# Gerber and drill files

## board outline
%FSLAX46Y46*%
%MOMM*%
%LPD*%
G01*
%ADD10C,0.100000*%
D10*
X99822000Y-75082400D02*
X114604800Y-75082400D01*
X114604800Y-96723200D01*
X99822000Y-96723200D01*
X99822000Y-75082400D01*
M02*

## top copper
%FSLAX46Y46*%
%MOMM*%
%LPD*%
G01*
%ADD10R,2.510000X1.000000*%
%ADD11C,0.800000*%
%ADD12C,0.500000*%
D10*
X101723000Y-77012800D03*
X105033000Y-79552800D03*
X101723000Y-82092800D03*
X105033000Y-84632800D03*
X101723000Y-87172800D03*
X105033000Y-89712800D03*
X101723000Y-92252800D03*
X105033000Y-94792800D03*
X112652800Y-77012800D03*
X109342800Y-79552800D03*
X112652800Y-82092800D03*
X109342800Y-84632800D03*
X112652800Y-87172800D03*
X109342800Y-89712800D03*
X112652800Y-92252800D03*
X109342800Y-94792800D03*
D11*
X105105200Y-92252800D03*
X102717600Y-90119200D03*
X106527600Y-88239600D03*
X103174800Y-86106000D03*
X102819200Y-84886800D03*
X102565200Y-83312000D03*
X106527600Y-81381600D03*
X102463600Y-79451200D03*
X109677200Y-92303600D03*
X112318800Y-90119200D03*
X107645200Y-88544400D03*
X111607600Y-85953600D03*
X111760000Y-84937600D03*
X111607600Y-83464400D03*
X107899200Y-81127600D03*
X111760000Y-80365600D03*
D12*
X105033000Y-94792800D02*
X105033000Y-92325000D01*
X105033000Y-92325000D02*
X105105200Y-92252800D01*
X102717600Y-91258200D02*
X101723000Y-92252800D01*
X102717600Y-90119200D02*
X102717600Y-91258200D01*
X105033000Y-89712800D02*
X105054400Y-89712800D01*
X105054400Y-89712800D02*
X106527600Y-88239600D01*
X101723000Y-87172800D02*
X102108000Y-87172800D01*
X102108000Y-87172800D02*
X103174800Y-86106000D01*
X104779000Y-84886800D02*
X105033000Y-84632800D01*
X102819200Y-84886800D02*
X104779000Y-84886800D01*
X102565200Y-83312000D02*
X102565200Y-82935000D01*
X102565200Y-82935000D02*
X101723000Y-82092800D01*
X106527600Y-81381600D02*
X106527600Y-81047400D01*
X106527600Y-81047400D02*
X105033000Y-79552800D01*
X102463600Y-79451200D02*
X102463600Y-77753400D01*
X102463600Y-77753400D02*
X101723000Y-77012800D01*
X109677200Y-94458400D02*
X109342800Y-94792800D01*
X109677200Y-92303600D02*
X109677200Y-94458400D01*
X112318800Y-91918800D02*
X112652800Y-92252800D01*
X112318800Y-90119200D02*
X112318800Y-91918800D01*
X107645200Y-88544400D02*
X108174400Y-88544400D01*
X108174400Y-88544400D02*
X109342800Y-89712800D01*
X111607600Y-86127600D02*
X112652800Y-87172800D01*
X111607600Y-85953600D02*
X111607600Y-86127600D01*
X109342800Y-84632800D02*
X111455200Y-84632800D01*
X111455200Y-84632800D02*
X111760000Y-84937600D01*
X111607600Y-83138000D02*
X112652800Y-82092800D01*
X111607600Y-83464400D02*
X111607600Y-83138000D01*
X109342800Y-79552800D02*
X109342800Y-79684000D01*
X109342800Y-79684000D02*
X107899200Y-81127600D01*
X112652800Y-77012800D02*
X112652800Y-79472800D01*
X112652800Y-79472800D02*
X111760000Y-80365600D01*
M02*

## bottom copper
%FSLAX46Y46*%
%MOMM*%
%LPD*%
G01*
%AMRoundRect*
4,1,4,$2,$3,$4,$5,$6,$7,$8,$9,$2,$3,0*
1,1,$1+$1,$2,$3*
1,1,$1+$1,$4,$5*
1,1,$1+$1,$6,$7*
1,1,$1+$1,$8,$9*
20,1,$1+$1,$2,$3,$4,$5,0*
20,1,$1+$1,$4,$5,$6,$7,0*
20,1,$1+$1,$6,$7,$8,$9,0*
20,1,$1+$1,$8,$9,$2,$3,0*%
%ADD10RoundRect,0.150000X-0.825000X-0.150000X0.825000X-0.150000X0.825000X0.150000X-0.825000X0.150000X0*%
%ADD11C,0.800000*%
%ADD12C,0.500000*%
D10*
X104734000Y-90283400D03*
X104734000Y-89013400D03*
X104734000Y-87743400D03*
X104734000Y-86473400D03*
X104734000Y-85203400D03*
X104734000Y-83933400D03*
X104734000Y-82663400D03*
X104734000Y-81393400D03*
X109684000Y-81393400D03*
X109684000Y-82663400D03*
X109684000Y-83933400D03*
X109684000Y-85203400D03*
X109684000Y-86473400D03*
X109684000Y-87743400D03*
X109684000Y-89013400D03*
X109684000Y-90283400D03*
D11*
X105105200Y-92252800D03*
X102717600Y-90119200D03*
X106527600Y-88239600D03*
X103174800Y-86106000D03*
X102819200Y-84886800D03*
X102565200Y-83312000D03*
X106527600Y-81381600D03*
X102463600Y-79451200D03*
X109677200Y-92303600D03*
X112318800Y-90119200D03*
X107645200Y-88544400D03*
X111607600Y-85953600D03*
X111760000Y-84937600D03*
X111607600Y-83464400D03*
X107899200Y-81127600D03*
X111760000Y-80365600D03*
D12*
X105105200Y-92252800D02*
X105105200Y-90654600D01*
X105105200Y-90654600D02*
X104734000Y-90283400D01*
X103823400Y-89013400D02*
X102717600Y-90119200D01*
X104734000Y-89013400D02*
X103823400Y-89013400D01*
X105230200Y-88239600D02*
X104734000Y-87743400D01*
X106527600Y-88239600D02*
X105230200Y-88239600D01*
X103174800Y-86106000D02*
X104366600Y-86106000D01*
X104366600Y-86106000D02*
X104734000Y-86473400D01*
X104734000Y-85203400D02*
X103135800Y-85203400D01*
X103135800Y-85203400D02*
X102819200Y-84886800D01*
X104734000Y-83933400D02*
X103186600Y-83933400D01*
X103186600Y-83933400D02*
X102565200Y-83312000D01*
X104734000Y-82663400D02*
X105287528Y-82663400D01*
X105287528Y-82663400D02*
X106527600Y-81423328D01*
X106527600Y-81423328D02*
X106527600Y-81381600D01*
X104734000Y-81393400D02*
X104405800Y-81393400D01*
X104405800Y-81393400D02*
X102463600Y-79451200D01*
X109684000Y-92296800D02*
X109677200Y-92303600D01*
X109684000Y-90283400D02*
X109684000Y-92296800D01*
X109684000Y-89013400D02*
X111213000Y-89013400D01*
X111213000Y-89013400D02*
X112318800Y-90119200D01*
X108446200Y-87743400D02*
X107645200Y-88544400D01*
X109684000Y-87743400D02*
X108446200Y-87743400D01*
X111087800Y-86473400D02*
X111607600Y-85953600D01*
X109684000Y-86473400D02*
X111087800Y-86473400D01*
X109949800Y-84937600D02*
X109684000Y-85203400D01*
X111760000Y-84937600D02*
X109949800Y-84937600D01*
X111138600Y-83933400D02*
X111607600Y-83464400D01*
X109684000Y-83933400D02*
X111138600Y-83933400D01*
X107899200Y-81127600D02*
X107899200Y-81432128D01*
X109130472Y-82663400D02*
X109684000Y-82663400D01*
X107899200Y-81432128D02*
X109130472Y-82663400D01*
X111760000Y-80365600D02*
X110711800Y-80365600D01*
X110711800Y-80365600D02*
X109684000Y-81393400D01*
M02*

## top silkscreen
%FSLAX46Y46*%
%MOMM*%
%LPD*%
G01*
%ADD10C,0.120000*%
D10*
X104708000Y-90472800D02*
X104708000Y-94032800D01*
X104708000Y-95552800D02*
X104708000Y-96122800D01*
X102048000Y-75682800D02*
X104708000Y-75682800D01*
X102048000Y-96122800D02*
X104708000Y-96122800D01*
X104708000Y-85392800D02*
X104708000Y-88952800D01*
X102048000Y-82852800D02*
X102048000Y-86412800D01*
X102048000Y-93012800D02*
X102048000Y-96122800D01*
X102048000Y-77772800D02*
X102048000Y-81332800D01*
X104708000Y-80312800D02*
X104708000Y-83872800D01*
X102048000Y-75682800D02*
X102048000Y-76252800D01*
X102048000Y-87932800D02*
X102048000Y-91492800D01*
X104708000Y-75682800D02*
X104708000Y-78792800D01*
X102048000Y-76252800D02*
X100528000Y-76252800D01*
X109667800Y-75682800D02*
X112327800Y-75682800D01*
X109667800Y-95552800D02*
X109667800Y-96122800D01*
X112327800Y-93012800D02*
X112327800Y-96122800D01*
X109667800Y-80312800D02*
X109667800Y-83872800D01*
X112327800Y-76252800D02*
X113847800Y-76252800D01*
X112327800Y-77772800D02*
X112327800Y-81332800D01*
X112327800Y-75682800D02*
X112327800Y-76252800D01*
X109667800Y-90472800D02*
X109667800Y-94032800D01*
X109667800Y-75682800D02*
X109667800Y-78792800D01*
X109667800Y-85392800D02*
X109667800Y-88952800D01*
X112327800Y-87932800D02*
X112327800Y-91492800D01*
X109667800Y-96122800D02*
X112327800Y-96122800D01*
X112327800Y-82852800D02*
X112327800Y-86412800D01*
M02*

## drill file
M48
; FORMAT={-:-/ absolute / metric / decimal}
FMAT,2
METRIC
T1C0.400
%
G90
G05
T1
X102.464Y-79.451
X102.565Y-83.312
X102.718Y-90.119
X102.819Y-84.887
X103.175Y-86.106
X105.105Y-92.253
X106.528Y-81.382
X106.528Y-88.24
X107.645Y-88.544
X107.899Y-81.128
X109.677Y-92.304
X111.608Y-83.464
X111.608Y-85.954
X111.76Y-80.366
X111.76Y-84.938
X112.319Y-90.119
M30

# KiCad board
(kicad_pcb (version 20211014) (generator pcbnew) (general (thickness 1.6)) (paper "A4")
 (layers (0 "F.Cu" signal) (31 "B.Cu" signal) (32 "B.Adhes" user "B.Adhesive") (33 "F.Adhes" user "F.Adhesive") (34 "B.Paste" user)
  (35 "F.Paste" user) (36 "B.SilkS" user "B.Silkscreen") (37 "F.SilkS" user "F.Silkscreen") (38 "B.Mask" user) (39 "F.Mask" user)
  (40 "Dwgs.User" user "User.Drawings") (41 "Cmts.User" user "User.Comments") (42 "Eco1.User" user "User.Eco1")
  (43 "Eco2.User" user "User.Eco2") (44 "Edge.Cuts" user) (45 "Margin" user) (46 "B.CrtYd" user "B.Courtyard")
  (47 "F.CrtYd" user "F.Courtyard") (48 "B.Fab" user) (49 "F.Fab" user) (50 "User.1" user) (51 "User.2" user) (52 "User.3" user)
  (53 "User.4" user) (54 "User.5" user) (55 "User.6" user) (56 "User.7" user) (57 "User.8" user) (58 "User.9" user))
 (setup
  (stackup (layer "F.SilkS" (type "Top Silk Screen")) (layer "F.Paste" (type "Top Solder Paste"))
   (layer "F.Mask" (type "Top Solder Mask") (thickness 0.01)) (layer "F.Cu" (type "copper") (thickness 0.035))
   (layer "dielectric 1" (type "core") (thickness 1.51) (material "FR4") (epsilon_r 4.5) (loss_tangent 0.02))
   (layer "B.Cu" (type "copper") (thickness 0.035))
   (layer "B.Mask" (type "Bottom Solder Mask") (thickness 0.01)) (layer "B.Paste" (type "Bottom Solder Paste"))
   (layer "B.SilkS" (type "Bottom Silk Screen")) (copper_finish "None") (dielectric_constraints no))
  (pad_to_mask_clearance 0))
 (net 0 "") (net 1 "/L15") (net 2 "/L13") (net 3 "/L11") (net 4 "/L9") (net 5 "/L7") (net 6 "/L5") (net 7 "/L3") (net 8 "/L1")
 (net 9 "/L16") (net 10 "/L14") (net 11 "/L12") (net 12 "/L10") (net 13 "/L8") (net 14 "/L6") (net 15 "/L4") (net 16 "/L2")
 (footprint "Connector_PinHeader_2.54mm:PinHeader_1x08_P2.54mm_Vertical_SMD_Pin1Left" (layer "F.Cu") (at 103.378 85.9028)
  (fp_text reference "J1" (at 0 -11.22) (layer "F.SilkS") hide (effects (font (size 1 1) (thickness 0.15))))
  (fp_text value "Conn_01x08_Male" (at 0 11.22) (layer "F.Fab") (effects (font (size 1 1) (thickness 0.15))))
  (fp_line (start 1.33 4.57) (end 1.33 8.13) (layer "F.SilkS") (width 0.12))
  (fp_line (start 1.33 9.65) (end 1.33 10.22) (layer "F.SilkS") (width 0.12))
  (fp_line (start -1.33 -10.22) (end 1.33 -10.22) (layer "F.SilkS") (width 0.12))
  (fp_line (start -1.33 10.22) (end 1.33 10.22) (layer "F.SilkS") (width 0.12))
  (fp_line (start 1.33 -0.51) (end 1.33 3.05) (layer "F.SilkS") (width 0.12))
  (fp_line (start -1.33 -3.05) (end -1.33 0.51) (layer "F.SilkS") (width 0.12))
  (fp_line (start -1.33 7.11) (end -1.33 10.22) (layer "F.SilkS") (width 0.12))
  (fp_line (start -1.33 -8.13) (end -1.33 -4.57) (layer "F.SilkS") (width 0.12))
  (fp_line (start 1.33 -5.59) (end 1.33 -2.03) (layer "F.SilkS") (width 0.12))
  (fp_line (start -1.33 -10.22) (end -1.33 -9.65) (layer "F.SilkS") (width 0.12))
  (fp_line (start -1.33 2.03) (end -1.33 5.59) (layer "F.SilkS") (width 0.12))
  (fp_line (start 1.33 -10.22) (end 1.33 -7.11) (layer "F.SilkS") (width 0.12))
  (fp_line (start -1.33 -9.65) (end -2.85 -9.65) (layer "F.SilkS") (width 0.12))
  (pad "1" smd rect (at -1.655 -8.89) (size 2.51 1) (layers "F.Cu" "F.Paste" "F.Mask") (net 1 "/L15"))
  (pad "2" smd rect (at 1.655 -6.35) (size 2.51 1) (layers "F.Cu" "F.Paste" "F.Mask") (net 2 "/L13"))
  (pad "3" smd rect (at -1.655 -3.81) (size 2.51 1) (layers "F.Cu" "F.Paste" "F.Mask") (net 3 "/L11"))
  (pad "4" smd rect (at 1.655 -1.27) (size 2.51 1) (layers "F.Cu" "F.Paste" "F.Mask") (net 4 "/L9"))
  (pad "5" smd rect (at -1.655 1.27) (size 2.51 1) (layers "F.Cu" "F.Paste" "F.Mask") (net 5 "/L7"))
  (pad "6" smd rect (at 1.655 3.81) (size 2.51 1) (layers "F.Cu" "F.Paste" "F.Mask") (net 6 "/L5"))
  (pad "7" smd rect (at -1.655 6.35) (size 2.51 1) (layers "F.Cu" "F.Paste" "F.Mask") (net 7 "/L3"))
  (pad "8" smd rect (at 1.655 8.89) (size 2.51 1) (layers "F.Cu" "F.Paste" "F.Mask") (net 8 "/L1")))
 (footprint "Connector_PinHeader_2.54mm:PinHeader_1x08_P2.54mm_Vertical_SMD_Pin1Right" (layer "F.Cu") (at 110.9978 85.9028)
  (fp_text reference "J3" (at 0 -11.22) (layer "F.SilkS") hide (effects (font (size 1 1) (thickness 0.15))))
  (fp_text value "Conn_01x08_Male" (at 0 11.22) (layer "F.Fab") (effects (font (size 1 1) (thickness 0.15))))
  (fp_line (start -1.33 -10.22) (end 1.33 -10.22) (layer "F.SilkS") (width 0.12))
  (fp_line (start -1.33 9.65) (end -1.33 10.22) (layer "F.SilkS") (width 0.12))
  (fp_line (start 1.33 7.11) (end 1.33 10.22) (layer "F.SilkS") (width 0.12))
  (fp_line (start -1.33 -5.59) (end -1.33 -2.03) (layer "F.SilkS") (width 0.12))
  (fp_line (start 1.33 -9.65) (end 2.85 -9.65) (layer "F.SilkS") (width 0.12))
  (fp_line (start 1.33 -8.13) (end 1.33 -4.57) (layer "F.SilkS") (width 0.12))
  (fp_line (start 1.33 -10.22) (end 1.33 -9.65) (layer "F.SilkS") (width 0.12))
  (fp_line (start -1.33 4.57) (end -1.33 8.13) (layer "F.SilkS") (width 0.12))
  (fp_line (start -1.33 -10.22) (end -1.33 -7.11) (layer "F.SilkS") (width 0.12))
  (fp_line (start -1.33 -0.51) (end -1.33 3.05) (layer "F.SilkS") (width 0.12))
  (fp_line (start 1.33 2.03) (end 1.33 5.59) (layer "F.SilkS") (width 0.12))
  (fp_line (start -1.33 10.22) (end 1.33 10.22) (layer "F.SilkS") (width 0.12))
  (fp_line (start 1.33 -3.05) (end 1.33 0.51) (layer "F.SilkS") (width 0.12))
  (pad "1" smd rect (at 1.655 -8.89) (size 2.51 1) (layers "F.Cu" "F.Paste" "F.Mask") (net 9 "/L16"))
  (pad "2" smd rect (at -1.655 -6.35) (size 2.51 1) (layers "F.Cu" "F.Paste" "F.Mask") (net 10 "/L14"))
  (pad "3" smd rect (at 1.655 -3.81) (size 2.51 1) (layers "F.Cu" "F.Paste" "F.Mask") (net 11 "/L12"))
  (pad "4" smd rect (at -1.655 -1.27) (size 2.51 1) (layers "F.Cu" "F.Paste" "F.Mask") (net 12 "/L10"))
  (pad "5" smd rect (at 1.655 1.27) (size 2.51 1) (layers "F.Cu" "F.Paste" "F.Mask") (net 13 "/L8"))
  (pad "6" smd rect (at -1.655 3.81) (size 2.51 1) (layers "F.Cu" "F.Paste" "F.Mask") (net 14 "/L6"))
  (pad "7" smd rect (at 1.655 6.35) (size 2.51 1) (layers "F.Cu" "F.Paste" "F.Mask") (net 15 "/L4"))
  (pad "8" smd rect (at -1.655 8.89) (size 2.51 1) (layers "F.Cu" "F.Paste" "F.Mask") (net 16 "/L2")))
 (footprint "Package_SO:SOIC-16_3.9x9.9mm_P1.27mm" (layer "B.Cu") (at 107.209 85.8384)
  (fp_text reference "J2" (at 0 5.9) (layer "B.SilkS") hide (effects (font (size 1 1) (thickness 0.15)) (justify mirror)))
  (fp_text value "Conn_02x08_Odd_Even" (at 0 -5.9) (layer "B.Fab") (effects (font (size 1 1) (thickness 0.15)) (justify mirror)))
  (pad "1" smd roundrect (at -2.475 4.445) (size 1.95 0.6) (layers "B.Cu" "B.Paste" "B.Mask") (roundrect_rratio 0.25) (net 8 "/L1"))
  (pad "2" smd roundrect (at -2.475 3.175) (size 1.95 0.6) (layers "B.Cu" "B.Paste" "B.Mask") (roundrect_rratio 0.25) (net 7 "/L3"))
  (pad "3" smd roundrect (at -2.475 1.905) (size 1.95 0.6) (layers "B.Cu" "B.Paste" "B.Mask") (roundrect_rratio 0.25) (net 6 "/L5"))
  (pad "4" smd roundrect (at -2.475 0.635) (size 1.95 0.6) (layers "B.Cu" "B.Paste" "B.Mask") (roundrect_rratio 0.25) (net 5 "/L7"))
  (pad "5" smd roundrect (at -2.475 -0.635) (size 1.95 0.6) (layers "B.Cu" "B.Paste" "B.Mask") (roundrect_rratio 0.25) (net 4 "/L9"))
  (pad "6" smd roundrect (at -2.475 -1.905) (size 1.95 0.6) (layers "B.Cu" "B.Paste" "B.Mask") (roundrect_rratio 0.25) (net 3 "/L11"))
  (pad "7" smd roundrect (at -2.475 -3.175) (size 1.95 0.6) (layers "B.Cu" "B.Paste" "B.Mask") (roundrect_rratio 0.25) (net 2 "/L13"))
  (pad "8" smd roundrect (at -2.475 -4.445) (size 1.95 0.6) (layers "B.Cu" "B.Paste" "B.Mask") (roundrect_rratio 0.25) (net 1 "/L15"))
  (pad "9" smd roundrect (at 2.475 -4.445) (size 1.95 0.6) (layers "B.Cu" "B.Paste" "B.Mask") (roundrect_rratio 0.25) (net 9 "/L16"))
  (pad "10" smd roundrect (at 2.475 -3.175) (size 1.95 0.6) (layers "B.Cu" "B.Paste" "B.Mask") (roundrect_rratio 0.25) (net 10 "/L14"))
  (pad "11" smd roundrect (at 2.475 -1.905) (size 1.95 0.6) (layers "B.Cu" "B.Paste" "B.Mask") (roundrect_rratio 0.25) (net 11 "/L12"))
  (pad "12" smd roundrect (at 2.475 -0.635) (size 1.95 0.6) (layers "B.Cu" "B.Paste" "B.Mask") (roundrect_rratio 0.25) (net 12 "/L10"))
  (pad "13" smd roundrect (at 2.475 0.635) (size 1.95 0.6) (layers "B.Cu" "B.Paste" "B.Mask") (roundrect_rratio 0.25) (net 13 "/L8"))
  (pad "14" smd roundrect (at 2.475 1.905) (size 1.95 0.6) (layers "B.Cu" "B.Paste" "B.Mask") (roundrect_rratio 0.25) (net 14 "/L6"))
  (pad "15" smd roundrect (at 2.475 3.175) (size 1.95 0.6) (layers "B.Cu" "B.Paste" "B.Mask") (roundrect_rratio 0.25) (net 15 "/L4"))
  (pad "16" smd roundrect (at 2.475 4.445) (size 1.95 0.6) (layers "B.Cu" "B.Paste" "B.Mask") (roundrect_rratio 0.25) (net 16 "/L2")))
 (gr_rect (start 99.822 75.0824) (end 114.6048 96.7232) (layer "Edge.Cuts") (width 0.1) (fill none))
 (segment (start 105.033 94.7928) (end 105.033 92.325) (width 0.5) (layer "F.Cu") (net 8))
 (segment (start 105.033 92.325) (end 105.1052 92.2528) (width 0.5) (layer "F.Cu") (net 8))
 (via (at 105.1052 92.2528) (size 0.8) (drill 0.4) (layers "F.Cu" "B.Cu") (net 8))
 (segment (start 105.1052 92.2528) (end 105.1052 90.6546) (width 0.5) (layer "B.Cu") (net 8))
 (segment (start 105.1052 90.6546) (end 104.734 90.2834) (width 0.5) (layer "B.Cu") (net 8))
 (segment (start 102.7176 91.2582) (end 101.723 92.2528) (width 0.5) (layer "F.Cu") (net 7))
 (segment (start 102.7176 90.1192) (end 102.7176 91.2582) (width 0.5) (layer "F.Cu") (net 7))
 (via (at 102.7176 90.1192) (size 0.8) (drill 0.4) (layers "F.Cu" "B.Cu") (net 7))
 (segment (start 103.8234 89.0134) (end 102.7176 90.1192) (width 0.5) (layer "B.Cu") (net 7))
 (segment (start 104.734 89.0134) (end 103.8234 89.0134) (width 0.5) (layer "B.Cu") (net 7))
 (segment (start 105.033 89.7128) (end 105.0544 89.7128) (width 0.5) (layer "F.Cu") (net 6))
 (segment (start 105.0544 89.7128) (end 106.5276 88.2396) (width 0.5) (layer "F.Cu") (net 6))
 (via (at 106.5276 88.2396) (size 0.8) (drill 0.4) (layers "F.Cu" "B.Cu") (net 6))
 (segment (start 105.2302 88.2396) (end 104.734 87.7434) (width 0.5) (layer "B.Cu") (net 6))
 (segment (start 106.5276 88.2396) (end 105.2302 88.2396) (width 0.5) (layer "B.Cu") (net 6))
 (segment (start 101.723 87.1728) (end 102.108 87.1728) (width 0.5) (layer "F.Cu") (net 5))
 (segment (start 102.108 87.1728) (end 103.1748 86.106) (width 0.5) (layer "F.Cu") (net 5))
 (via (at 103.1748 86.106) (size 0.8) (drill 0.4) (layers "F.Cu" "B.Cu") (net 5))
 (segment (start 103.1748 86.106) (end 104.3666 86.106) (width 0.5) (layer "B.Cu") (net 5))
 (segment (start 104.3666 86.106) (end 104.734 86.4734) (width 0.5) (layer "B.Cu") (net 5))
 (segment (start 104.779 84.8868) (end 105.033 84.6328) (width 0.5) (layer "F.Cu") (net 4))
 (segment (start 102.8192 84.8868) (end 104.779 84.8868) (width 0.5) (layer "F.Cu") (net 4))
 (via (at 102.8192 84.8868) (size 0.8) (drill 0.4) (layers "F.Cu" "B.Cu") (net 4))
 (segment (start 104.734 85.2034) (end 103.1358 85.2034) (width 0.5) (layer "B.Cu") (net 4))
 (segment (start 103.1358 85.2034) (end 102.8192 84.8868) (width 0.5) (layer "B.Cu") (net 4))
 (segment (start 102.5652 83.312) (end 102.5652 82.935) (width 0.5) (layer "F.Cu") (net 3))
 (segment (start 102.5652 82.935) (end 101.723 82.0928) (width 0.5) (layer "F.Cu") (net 3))
 (via (at 102.5652 83.312) (size 0.8) (drill 0.4) (layers "F.Cu" "B.Cu") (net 3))
 (segment (start 104.734 83.9334) (end 103.1866 83.9334) (width 0.5) (layer "B.Cu") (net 3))
 (segment (start 103.1866 83.9334) (end 102.5652 83.312) (width 0.5) (layer "B.Cu") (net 3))
 (segment (start 106.5276 81.3816) (end 106.5276 81.0474) (width 0.5) (layer "F.Cu") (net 2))
 (segment (start 106.5276 81.0474) (end 105.033 79.5528) (width 0.5) (layer "F.Cu") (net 2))
 (via (at 106.5276 81.3816) (size 0.8) (drill 0.4) (layers "F.Cu" "B.Cu") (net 2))
 (segment (start 104.734 82.6634) (end 105.287528 82.6634) (width 0.5) (layer "B.Cu") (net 2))
 (segment (start 105.287528 82.6634) (end 106.5276 81.423328) (width 0.5) (layer "B.Cu") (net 2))
 (segment (start 106.5276 81.423328) (end 106.5276 81.3816) (width 0.5) (layer "B.Cu") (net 2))
 (segment (start 102.4636 79.4512) (end 102.4636 77.7534) (width 0.5) (layer "F.Cu") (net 1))
 (segment (start 102.4636 77.7534) (end 101.723 77.0128) (width 0.5) (layer "F.Cu") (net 1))
 (via (at 102.4636 79.4512) (size 0.8) (drill 0.4) (layers "F.Cu" "B.Cu") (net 1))
 (segment (start 104.734 81.3934) (end 104.4058 81.3934) (width 0.5) (layer "B.Cu") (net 1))
 (segment (start 104.4058 81.3934) (end 102.4636 79.4512) (width 0.5) (layer "B.Cu") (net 1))
 (segment (start 109.6772 94.4584) (end 109.3428 94.7928) (width 0.5) (layer "F.Cu") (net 16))
 (segment (start 109.6772 92.3036) (end 109.6772 94.4584) (width 0.5) (layer "F.Cu") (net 16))
 (via (at 109.6772 92.3036) (size 0.8) (drill 0.4) (layers "F.Cu" "B.Cu") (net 16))
 (segment (start 109.684 92.2968) (end 109.6772 92.3036) (width 0.5) (layer "B.Cu") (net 16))
 (segment (start 109.684 90.2834) (end 109.684 92.2968) (width 0.5) (layer "B.Cu") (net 16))
 (segment (start 112.3188 91.9188) (end 112.6528 92.2528) (width 0.5) (layer "F.Cu") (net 15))
 (segment (start 112.3188 90.1192) (end 112.3188 91.9188) (width 0.5) (layer "F.Cu") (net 15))
 (via (at 112.3188 90.1192) (size 0.8) (drill 0.4) (layers "F.Cu" "B.Cu") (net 15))
 (segment (start 109.684 89.0134) (end 111.213 89.0134) (width 0.5) (layer "B.Cu") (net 15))
 (segment (start 111.213 89.0134) (end 112.3188 90.1192) (width 0.5) (layer "B.Cu") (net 15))
 (segment (start 107.6452 88.5444) (end 108.1744 88.5444) (width 0.5) (layer "F.Cu") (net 14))
 (segment (start 108.1744 88.5444) (end 109.3428 89.7128) (width 0.5) (layer "F.Cu") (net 14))
 (via (at 107.6452 88.5444) (size 0.8) (drill 0.4) (layers "F.Cu" "B.Cu") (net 14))
 (segment (start 108.4462 87.7434) (end 107.6452 88.5444) (width 0.5) (layer "B.Cu") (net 14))
 (segment (start 109.684 87.7434) (end 108.4462 87.7434) (width 0.5) (layer "B.Cu") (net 14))
 (segment (start 111.6076 86.1276) (end 112.6528 87.1728) (width 0.5) (layer "F.Cu") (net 13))
 (segment (start 111.6076 85.9536) (end 111.6076 86.1276) (width 0.5) (layer "F.Cu") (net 13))
 (via (at 111.6076 85.9536) (size 0.8) (drill 0.4) (layers "F.Cu" "B.Cu") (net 13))
 (segment (start 111.0878 86.4734) (end 111.6076 85.9536) (width 0.5) (layer "B.Cu") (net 13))
 (segment (start 109.684 86.4734) (end 111.0878 86.4734) (width 0.5) (layer "B.Cu") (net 13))
 (segment (start 109.3428 84.6328) (end 111.4552 84.6328) (width 0.5) (layer "F.Cu") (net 12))
 (segment (start 111.4552 84.6328) (end 111.76 84.9376) (width 0.5) (layer "F.Cu") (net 12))
 (via (at 111.76 84.9376) (size 0.8) (drill 0.4) (layers "F.Cu" "B.Cu") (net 12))
 (segment (start 109.9498 84.9376) (end 109.684 85.2034) (width 0.5) (layer "B.Cu") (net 12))
 (segment (start 111.76 84.9376) (end 109.9498 84.9376) (width 0.5) (layer "B.Cu") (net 12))
 (segment (start 111.6076 83.138) (end 112.6528 82.0928) (width 0.5) (layer "F.Cu") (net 11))
 (segment (start 111.6076 83.4644) (end 111.6076 83.138) (width 0.5) (layer "F.Cu") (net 11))
 (via (at 111.6076 83.4644) (size 0.8) (drill 0.4) (layers "F.Cu" "B.Cu") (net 11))
 (segment (start 111.1386 83.9334) (end 111.6076 83.4644) (width 0.5) (layer "B.Cu") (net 11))
 (segment (start 109.684 83.9334) (end 111.1386 83.9334) (width 0.5) (layer "B.Cu") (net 11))
 (segment (start 109.3428 79.5528) (end 109.3428 79.684) (width 0.5) (layer "F.Cu") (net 10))
 (segment (start 109.3428 79.684) (end 107.8992 81.1276) (width 0.5) (layer "F.Cu") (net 10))
 (via (at 107.8992 81.1276) (size 0.8) (drill 0.4) (layers "F.Cu" "B.Cu") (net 10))
 (segment (start 107.8992 81.1276) (end 107.8992 81.432128) (width 0.5) (layer "B.Cu") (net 10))
 (segment (start 109.130472 82.6634) (end 109.684 82.6634) (width 0.5) (layer "B.Cu") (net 10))
 (segment (start 107.8992 81.432128) (end 109.130472 82.6634) (width 0.5) (layer "B.Cu") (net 10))
 (segment (start 112.6528 77.0128) (end 112.6528 79.4728) (width 0.5) (layer "F.Cu") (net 9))
 (segment (start 112.6528 79.4728) (end 111.76 80.3656) (width 0.5) (layer "F.Cu") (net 9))
 (via (at 111.76 80.3656) (size 0.8) (drill 0.4) (layers "F.Cu" "B.Cu") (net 9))
 (segment (start 111.76 80.3656) (end 110.7118 80.3656) (width 0.5) (layer "B.Cu") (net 9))
 (segment (start 110.7118 80.3656) (end 109.684 81.3934) (width 0.5) (layer "B.Cu") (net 9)))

